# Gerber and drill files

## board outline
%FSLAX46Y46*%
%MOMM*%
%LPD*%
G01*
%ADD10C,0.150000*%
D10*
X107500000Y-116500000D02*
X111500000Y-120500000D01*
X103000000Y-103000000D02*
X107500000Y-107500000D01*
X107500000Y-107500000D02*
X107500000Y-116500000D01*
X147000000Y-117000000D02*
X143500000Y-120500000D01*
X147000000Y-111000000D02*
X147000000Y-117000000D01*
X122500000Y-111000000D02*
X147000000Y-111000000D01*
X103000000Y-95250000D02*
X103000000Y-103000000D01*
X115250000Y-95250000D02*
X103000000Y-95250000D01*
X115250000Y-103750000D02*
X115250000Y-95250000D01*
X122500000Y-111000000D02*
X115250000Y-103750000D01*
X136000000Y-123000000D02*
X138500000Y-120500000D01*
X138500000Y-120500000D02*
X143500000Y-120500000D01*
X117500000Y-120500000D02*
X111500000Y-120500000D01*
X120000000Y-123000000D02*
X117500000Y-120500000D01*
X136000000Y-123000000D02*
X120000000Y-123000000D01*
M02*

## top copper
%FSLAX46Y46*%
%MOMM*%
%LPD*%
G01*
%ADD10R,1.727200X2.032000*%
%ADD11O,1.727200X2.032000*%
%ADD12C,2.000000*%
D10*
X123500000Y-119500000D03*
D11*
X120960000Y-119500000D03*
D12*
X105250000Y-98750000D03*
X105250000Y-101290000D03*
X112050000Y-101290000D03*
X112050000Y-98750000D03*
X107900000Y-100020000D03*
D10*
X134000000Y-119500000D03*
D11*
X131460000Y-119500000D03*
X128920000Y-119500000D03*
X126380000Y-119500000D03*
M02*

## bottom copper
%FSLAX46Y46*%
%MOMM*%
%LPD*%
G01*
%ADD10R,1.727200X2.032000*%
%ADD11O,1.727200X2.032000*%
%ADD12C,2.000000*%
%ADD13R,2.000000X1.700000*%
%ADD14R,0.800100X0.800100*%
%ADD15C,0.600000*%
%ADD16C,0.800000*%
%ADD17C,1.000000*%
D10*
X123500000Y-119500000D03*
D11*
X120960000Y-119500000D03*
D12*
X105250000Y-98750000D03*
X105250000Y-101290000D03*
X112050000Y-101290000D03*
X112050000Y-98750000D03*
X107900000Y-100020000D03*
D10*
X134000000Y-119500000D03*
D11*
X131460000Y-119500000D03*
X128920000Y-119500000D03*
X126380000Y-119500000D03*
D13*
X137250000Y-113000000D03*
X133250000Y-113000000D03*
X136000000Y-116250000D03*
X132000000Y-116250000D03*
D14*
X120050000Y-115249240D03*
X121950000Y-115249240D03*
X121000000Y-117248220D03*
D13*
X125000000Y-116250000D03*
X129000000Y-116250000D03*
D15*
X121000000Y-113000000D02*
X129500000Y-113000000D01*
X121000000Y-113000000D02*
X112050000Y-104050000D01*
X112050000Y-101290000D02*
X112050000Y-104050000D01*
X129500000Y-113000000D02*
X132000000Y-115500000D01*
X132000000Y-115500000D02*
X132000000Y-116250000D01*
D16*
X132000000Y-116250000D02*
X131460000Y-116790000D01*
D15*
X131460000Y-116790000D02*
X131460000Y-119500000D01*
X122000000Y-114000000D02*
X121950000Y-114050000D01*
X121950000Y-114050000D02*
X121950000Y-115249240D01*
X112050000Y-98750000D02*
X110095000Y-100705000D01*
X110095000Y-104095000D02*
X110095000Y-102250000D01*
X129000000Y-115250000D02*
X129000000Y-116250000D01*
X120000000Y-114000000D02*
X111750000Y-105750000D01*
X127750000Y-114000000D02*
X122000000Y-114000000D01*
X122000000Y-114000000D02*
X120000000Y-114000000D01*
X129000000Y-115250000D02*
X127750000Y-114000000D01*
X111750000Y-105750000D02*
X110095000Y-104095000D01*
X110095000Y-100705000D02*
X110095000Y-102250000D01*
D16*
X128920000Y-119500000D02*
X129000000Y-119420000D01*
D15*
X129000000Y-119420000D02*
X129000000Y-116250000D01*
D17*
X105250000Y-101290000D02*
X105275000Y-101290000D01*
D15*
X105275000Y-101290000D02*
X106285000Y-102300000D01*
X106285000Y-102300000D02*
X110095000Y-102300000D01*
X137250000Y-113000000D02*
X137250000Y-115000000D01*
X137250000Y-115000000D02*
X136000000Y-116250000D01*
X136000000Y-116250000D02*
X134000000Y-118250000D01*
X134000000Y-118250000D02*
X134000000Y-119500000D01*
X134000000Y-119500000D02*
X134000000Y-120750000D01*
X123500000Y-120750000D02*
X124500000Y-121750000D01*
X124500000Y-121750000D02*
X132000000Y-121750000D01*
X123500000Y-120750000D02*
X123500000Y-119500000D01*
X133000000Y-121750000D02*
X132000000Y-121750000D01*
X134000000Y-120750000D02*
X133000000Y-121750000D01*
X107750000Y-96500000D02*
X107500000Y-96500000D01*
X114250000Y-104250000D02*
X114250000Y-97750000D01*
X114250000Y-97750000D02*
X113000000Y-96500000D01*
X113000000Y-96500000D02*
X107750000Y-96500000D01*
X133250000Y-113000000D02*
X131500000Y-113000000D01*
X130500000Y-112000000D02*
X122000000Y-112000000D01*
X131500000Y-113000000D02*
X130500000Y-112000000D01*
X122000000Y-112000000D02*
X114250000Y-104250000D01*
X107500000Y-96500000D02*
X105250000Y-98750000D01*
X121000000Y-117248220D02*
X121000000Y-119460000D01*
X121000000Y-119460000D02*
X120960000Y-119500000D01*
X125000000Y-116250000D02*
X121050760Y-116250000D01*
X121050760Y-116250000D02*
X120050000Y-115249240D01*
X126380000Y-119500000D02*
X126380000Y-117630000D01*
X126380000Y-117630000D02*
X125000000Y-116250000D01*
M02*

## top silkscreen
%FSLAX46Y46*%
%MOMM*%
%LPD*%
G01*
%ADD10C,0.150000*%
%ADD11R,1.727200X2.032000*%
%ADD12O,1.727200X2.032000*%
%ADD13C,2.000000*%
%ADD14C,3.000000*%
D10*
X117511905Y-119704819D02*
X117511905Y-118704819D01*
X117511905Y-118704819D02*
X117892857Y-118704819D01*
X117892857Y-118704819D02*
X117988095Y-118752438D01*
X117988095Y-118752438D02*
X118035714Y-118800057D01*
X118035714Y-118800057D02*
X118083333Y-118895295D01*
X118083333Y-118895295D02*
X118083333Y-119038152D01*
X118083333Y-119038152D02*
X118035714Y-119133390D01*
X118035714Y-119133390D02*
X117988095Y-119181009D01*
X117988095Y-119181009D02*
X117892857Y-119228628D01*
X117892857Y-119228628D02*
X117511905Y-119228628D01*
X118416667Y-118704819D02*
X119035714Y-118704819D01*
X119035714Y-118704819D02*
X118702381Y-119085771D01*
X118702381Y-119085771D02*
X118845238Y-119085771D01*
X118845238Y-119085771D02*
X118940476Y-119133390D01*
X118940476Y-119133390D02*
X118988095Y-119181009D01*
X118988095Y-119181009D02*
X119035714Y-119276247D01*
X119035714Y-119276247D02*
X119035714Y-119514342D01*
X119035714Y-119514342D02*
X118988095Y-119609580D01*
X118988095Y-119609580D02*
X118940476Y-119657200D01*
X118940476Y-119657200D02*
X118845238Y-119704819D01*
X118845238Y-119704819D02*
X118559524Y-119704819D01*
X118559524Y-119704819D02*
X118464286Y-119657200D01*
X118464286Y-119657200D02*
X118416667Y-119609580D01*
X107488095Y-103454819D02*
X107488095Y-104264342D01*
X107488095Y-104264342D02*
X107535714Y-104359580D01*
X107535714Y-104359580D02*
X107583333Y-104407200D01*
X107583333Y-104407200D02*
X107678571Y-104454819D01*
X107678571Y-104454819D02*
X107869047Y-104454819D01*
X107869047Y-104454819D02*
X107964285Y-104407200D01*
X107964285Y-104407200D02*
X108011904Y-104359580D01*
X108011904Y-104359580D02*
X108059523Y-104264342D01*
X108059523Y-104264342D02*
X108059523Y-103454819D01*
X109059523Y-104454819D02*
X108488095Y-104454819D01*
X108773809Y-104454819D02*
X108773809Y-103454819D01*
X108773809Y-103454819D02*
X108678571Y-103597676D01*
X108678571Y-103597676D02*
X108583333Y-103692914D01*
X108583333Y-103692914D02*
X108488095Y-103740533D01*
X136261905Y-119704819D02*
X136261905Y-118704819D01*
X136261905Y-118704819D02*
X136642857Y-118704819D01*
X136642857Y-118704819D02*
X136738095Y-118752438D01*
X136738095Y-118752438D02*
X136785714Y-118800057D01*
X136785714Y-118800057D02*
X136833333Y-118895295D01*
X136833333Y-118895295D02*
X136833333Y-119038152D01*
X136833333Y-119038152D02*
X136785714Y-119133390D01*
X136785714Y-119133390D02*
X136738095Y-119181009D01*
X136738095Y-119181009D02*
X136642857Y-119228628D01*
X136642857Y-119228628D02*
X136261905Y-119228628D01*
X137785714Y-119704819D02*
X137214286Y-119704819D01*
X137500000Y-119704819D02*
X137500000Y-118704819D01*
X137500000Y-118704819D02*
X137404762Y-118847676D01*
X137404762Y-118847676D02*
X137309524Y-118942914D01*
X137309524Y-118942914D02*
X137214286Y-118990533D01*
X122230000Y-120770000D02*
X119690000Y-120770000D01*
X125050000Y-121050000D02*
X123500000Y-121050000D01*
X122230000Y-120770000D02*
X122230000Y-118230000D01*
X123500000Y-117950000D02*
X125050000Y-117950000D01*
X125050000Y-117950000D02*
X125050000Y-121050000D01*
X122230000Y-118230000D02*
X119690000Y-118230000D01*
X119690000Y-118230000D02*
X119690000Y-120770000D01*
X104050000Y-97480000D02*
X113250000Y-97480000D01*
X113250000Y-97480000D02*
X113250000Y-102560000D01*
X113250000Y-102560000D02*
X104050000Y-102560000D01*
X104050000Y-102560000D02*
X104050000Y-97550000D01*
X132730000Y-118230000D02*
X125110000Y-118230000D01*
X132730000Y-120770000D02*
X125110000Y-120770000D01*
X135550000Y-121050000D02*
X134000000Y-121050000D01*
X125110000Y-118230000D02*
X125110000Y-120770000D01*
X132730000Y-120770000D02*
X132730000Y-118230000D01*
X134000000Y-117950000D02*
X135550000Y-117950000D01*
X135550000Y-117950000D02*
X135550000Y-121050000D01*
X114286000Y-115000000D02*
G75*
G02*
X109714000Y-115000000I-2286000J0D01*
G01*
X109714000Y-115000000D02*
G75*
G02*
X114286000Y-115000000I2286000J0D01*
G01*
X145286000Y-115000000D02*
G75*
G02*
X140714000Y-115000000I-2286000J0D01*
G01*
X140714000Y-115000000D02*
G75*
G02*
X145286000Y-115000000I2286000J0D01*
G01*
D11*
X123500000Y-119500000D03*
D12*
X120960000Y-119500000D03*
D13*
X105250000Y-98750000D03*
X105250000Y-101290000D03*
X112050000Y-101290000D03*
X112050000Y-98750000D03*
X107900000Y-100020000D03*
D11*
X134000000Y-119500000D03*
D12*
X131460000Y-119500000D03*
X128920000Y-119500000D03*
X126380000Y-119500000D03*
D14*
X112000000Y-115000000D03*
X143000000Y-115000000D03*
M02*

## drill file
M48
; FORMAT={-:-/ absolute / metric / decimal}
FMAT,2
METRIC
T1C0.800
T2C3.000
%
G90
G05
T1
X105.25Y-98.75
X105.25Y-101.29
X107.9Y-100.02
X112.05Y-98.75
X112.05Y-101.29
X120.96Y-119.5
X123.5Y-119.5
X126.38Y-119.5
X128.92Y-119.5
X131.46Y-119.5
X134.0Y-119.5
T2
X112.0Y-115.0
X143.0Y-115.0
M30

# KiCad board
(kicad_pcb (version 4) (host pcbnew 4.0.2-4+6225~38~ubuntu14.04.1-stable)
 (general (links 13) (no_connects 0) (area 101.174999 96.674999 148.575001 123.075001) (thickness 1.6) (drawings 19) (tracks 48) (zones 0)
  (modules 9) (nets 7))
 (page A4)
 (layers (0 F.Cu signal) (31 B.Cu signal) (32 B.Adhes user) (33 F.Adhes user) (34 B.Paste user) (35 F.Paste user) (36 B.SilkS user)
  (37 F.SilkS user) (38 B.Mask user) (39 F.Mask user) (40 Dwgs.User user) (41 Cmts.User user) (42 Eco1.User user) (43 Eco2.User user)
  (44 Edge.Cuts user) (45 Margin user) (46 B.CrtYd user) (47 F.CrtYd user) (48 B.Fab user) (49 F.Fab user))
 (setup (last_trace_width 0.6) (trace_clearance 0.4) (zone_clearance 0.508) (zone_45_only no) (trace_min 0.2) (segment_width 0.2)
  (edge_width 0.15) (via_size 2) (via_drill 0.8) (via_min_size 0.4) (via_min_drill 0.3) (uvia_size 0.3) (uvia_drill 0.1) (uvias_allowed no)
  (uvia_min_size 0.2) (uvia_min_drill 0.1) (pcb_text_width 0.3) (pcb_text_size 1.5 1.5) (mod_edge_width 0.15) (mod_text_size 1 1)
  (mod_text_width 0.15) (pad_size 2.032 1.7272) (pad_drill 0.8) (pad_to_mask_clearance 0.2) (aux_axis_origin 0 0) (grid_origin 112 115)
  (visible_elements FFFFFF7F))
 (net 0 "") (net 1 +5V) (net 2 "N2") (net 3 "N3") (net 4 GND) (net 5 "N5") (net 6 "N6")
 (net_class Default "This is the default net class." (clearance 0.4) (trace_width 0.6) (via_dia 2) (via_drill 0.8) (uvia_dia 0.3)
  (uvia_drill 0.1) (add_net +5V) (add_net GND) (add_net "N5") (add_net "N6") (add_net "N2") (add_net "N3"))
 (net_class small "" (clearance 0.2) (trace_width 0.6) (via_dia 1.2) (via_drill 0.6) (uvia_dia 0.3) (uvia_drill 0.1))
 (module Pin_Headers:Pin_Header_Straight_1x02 (layer F.Cu) (at 123.5 119.5 270)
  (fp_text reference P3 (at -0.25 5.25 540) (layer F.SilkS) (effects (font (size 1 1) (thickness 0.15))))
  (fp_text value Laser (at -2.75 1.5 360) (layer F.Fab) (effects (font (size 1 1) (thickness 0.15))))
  (fp_line (start 1.27 1.27) (end 1.27 3.81) (layer F.SilkS) (width 0.15))
  (fp_line (start 1.55 -1.55) (end 1.55 0) (layer F.SilkS) (width 0.15))
  (fp_line (start 1.27 1.27) (end -1.27 1.27) (layer F.SilkS) (width 0.15))
  (fp_line (start -1.55 0) (end -1.55 -1.55) (layer F.SilkS) (width 0.15))
  (fp_line (start -1.55 -1.55) (end 1.55 -1.55) (layer F.SilkS) (width 0.15))
  (fp_line (start -1.27 1.27) (end -1.27 3.81) (layer F.SilkS) (width 0.15))
  (fp_line (start -1.27 3.81) (end 1.27 3.81) (layer F.SilkS) (width 0.15))
  (pad 1 thru_hole rect (at 0 0 270) (size 2.032 1.7272) (drill 0.8) (layers *.Cu *.Mask F.SilkS) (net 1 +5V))
  (pad 2 thru_hole oval (at 0 2.54 270) (size 2.032 1.7272) (drill 0.8) (layers *.Cu *.Mask F.SilkS) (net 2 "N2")))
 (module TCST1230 (layer F.Cu) (at 105.25 98.75)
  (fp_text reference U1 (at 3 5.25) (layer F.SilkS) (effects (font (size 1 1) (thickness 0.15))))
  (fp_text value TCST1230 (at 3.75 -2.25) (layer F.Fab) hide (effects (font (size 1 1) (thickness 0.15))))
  (fp_line (start -1.2 -1.27) (end 8 -1.27) (layer F.SilkS) (width 0.15))
  (fp_line (start 8 -1.27) (end 8 3.81) (layer F.SilkS) (width 0.15))
  (fp_line (start 8 3.81) (end -1.2 3.81) (layer F.SilkS) (width 0.15))
  (fp_line (start -1.2 3.81) (end -1.2 -1.2) (layer F.SilkS) (width 0.15))
  (pad 1 thru_hole circle (at 0 0) (size 2 2) (drill 0.8) (layers *.Cu *.Mask F.SilkS) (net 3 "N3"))
  (pad 2 thru_hole circle (at 0 2.54) (size 2 2) (drill 0.8) (layers *.Cu *.Mask F.SilkS) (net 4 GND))
  (pad 3 thru_hole circle (at 6.8 2.54) (size 2 2) (drill 0.8) (layers *.Cu *.Mask F.SilkS) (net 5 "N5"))
  (pad 4 thru_hole circle (at 6.8 0) (size 2 2) (drill 0.8) (layers *.Cu *.Mask F.SilkS) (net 4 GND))
  (pad "" thru_hole circle (at 2.65 1.27) (size 2 2) (drill 0.8) (layers *.Cu *.Mask F.SilkS)))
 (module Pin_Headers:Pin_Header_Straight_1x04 (layer F.Cu) (at 134 119.5 270)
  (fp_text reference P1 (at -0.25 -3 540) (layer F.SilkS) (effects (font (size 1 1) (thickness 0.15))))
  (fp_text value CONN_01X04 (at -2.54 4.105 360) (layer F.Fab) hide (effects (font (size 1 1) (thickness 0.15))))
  (fp_line (start -1.27 1.27) (end -1.27 8.89) (layer F.SilkS) (width 0.15))
  (fp_line (start 1.27 1.27) (end 1.27 8.89) (layer F.SilkS) (width 0.15))
  (fp_line (start 1.55 -1.55) (end 1.55 0) (layer F.SilkS) (width 0.15))
  (fp_line (start -1.27 8.89) (end 1.27 8.89) (layer F.SilkS) (width 0.15))
  (fp_line (start 1.27 1.27) (end -1.27 1.27) (layer F.SilkS) (width 0.15))
  (fp_line (start -1.55 0) (end -1.55 -1.55) (layer F.SilkS) (width 0.15))
  (fp_line (start -1.55 -1.55) (end 1.55 -1.55) (layer F.SilkS) (width 0.15))
  (pad 1 thru_hole rect (at 0 0 270) (size 2.032 1.7272) (drill 0.8) (layers *.Cu *.Mask F.SilkS) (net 1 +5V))
  (pad 2 thru_hole oval (at 0 2.54 270) (size 2.032 1.7272) (drill 0.8) (layers *.Cu *.Mask F.SilkS) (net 5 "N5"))
  (pad 3 thru_hole oval (at 0 5.08 270) (size 2.032 1.7272) (drill 0.8) (layers *.Cu *.Mask F.SilkS) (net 4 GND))
  (pad 4 thru_hole oval (at 0 7.62 270) (size 2.032 1.7272) (drill 0.8) (layers *.Cu *.Mask F.SilkS) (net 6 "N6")))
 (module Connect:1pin (layer F.Cu) (at 112 115)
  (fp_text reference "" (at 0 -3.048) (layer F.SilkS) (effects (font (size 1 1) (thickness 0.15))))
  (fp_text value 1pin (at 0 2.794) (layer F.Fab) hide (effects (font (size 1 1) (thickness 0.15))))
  (fp_circle (center 0 0) (end 0 -2.286) (layer F.SilkS) (width 0.15))
  (pad "" np_thru_hole circle (at 0 0) (size 3 3) (drill 3) (layers *.Cu *.Mask F.SilkS)))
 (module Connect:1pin (layer F.Cu) (at 143 115)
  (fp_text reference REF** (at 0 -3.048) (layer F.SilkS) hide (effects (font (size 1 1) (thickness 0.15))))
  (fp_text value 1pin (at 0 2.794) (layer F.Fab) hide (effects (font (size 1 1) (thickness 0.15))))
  (fp_circle (center 0 0) (end 0 -2.286) (layer F.SilkS) (width 0.15))
  (pad "" np_thru_hole circle (at 0 0) (size 3 3) (drill 3) (layers *.Cu *.Mask F.SilkS)))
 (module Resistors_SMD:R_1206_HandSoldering (layer B.Cu) (at 135.25 113 180)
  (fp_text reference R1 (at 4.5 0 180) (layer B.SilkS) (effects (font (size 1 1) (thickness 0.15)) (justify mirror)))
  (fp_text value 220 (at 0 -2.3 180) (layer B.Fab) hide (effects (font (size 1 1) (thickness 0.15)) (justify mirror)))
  (pad 1 smd rect (at -2 0 180) (size 2 1.7) (layers B.Cu B.Paste B.Mask) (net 1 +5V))
  (pad 2 smd rect (at 2 0 180) (size 2 1.7) (layers B.Cu B.Paste B.Mask) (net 3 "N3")))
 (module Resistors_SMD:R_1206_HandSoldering (layer B.Cu) (at 134 116.25 180)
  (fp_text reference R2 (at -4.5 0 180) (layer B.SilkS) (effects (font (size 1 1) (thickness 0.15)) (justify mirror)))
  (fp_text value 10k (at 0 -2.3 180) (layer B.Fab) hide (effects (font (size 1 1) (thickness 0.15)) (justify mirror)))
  (pad 1 smd rect (at -2 0 180) (size 2 1.7) (layers B.Cu B.Paste B.Mask) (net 1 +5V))
  (pad 2 smd rect (at 2 0 180) (size 2 1.7) (layers B.Cu B.Paste B.Mask) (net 5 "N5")))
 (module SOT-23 (layer B.Cu) (at 121 116.25)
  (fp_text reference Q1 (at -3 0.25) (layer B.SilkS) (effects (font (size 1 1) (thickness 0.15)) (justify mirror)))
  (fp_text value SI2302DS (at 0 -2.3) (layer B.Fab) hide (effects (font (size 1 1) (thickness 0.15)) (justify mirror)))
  (pad 1 smd rect (at -0.95 -1.00076) (size 0.8001 0.8001) (layers B.Cu B.Paste B.Mask) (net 6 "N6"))
  (pad 2 smd rect (at 0.95 -1.00076) (size 0.8001 0.8001) (layers B.Cu B.Paste B.Mask) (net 4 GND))
  (pad 3 smd rect (at 0 0.99822) (size 0.8001 0.8001) (layers B.Cu B.Paste B.Mask) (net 2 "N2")))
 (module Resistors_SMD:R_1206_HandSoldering (layer B.Cu) (at 127 116.25)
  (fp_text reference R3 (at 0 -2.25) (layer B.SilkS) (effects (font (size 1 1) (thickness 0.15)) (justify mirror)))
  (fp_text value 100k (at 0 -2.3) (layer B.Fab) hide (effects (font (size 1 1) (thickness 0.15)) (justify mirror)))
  (pad 1 smd rect (at -2 0) (size 2 1.7) (layers B.Cu B.Paste B.Mask) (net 6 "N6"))
  (pad 2 smd rect (at 2 0) (size 2 1.7) (layers B.Cu B.Paste B.Mask) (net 4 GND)))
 (gr_line (start 107.5 116.5) (end 111.5 120.5) (angle 90) (layer Edge.Cuts) (width 0.15))
 (gr_line (start 103 103) (end 107.5 107.5) (angle 90) (layer Edge.Cuts) (width 0.15))
 (gr_line (start 107.5 107.5) (end 107.5 116.5) (angle 90) (layer Edge.Cuts) (width 0.15))
 (gr_line (start 147 117) (end 143.5 120.5) (angle 90) (layer Edge.Cuts) (width 0.15))
 (gr_line (start 147 111) (end 147 117) (angle 90) (layer Edge.Cuts) (width 0.15))
 (gr_line (start 122.5 111) (end 147 111) (angle 90) (layer Edge.Cuts) (width 0.15))
 (gr_line (start 103 95.25) (end 103 103) (angle 90) (layer Edge.Cuts) (width 0.15))
 (gr_line (start 115.25 95.25) (end 103 95.25) (angle 90) (layer Edge.Cuts) (width 0.15))
 (gr_line (start 115.25 103.75) (end 115.25 95.25) (angle 90) (layer Edge.Cuts) (width 0.15))
 (gr_line (start 122.5 111) (end 115.25 103.75) (angle 90) (layer Edge.Cuts) (width 0.15))
 (gr_line (start 136 123) (end 138.5 120.5) (angle 90) (layer Edge.Cuts) (width 0.15))
 (gr_line (start 138.5 120.5) (end 143.5 120.5) (angle 90) (layer Edge.Cuts) (width 0.15))
 (gr_line (start 117.5 120.5) (end 111.5 120.5) (angle 90) (layer Edge.Cuts) (width 0.15))
 (gr_line (start 120 123) (end 117.5 120.5) (angle 90) (layer Edge.Cuts) (width 0.15))
 (gr_line (start 136 123) (end 120 123) (angle 90) (layer Edge.Cuts) (width 0.15))
 (segment (start 121 113) (end 129.5 113) (width 0.6) (layer B.Cu) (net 5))
 (segment (start 121 113) (end 112.05 104.05) (width 0.6) (layer B.Cu) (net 5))
 (segment (start 112.05 101.29) (end 112.05 104.05) (width 0.6) (layer B.Cu) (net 5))
 (segment (start 129.5 113) (end 132 115.5) (width 0.6) (layer B.Cu) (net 5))
 (segment (start 132 115.5) (end 132 116.25) (width 0.6) (layer B.Cu) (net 5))
 (segment (start 132 116.25) (end 131.46 116.79) (width 0.8) (layer B.Cu) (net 5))
 (segment (start 131.46 116.79) (end 131.46 119.5) (width 0.6) (layer B.Cu) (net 5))
 (segment (start 122 114) (end 121.95 114.05) (width 0.6) (layer B.Cu) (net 4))
 (segment (start 121.95 114.05) (end 121.95 115.24924) (width 0.6) (layer B.Cu) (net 4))
 (segment (start 112.05 98.75) (end 110.095 100.705) (width 0.6) (layer B.Cu) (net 4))
 (segment (start 110.095 104.095) (end 110.095 102.25) (width 0.6) (layer B.Cu) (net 4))
 (segment (start 129 115.25) (end 129 116.25) (width 0.6) (layer B.Cu) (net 4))
 (segment (start 120 114) (end 111.75 105.75) (width 0.6) (layer B.Cu) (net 4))
 (segment (start 127.75 114) (end 122 114) (width 0.6) (layer B.Cu) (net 4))
 (segment (start 122 114) (end 120 114) (width 0.6) (layer B.Cu) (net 4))
 (segment (start 129 115.25) (end 127.75 114) (width 0.6) (layer B.Cu) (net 4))
 (segment (start 111.75 105.75) (end 110.095 104.095) (width 0.6) (layer B.Cu) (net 4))
 (segment (start 110.095 100.705) (end 110.095 102.25) (width 0.6) (layer B.Cu) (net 4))
 (segment (start 128.92 119.5) (end 129 119.42) (width 0.8) (layer B.Cu) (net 4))
 (segment (start 129 119.42) (end 129 116.25) (width 0.6) (layer B.Cu) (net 4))
 (segment (start 105.25 101.29) (end 105.275 101.29) (width 1) (layer B.Cu) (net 4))
 (segment (start 105.275 101.29) (end 106.285 102.3) (width 0.6) (layer B.Cu) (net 4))
 (segment (start 106.285 102.3) (end 110.095 102.3) (width 0.6) (layer B.Cu) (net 4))
 (segment (start 137.25 113) (end 137.25 115) (width 0.6) (layer B.Cu) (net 1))
 (segment (start 137.25 115) (end 136 116.25) (width 0.6) (layer B.Cu) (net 1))
 (segment (start 136 116.25) (end 134 118.25) (width 0.6) (layer B.Cu) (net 1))
 (segment (start 134 118.25) (end 134 119.5) (width 0.6) (layer B.Cu) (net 1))
 (segment (start 134 119.5) (end 134 120.75) (width 0.6) (layer B.Cu) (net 1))
 (segment (start 123.5 120.75) (end 124.5 121.75) (width 0.6) (layer B.Cu) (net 1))
 (segment (start 124.5 121.75) (end 132 121.75) (width 0.6) (layer B.Cu) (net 1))
 (segment (start 123.5 120.75) (end 123.5 119.5) (width 0.6) (layer B.Cu) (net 1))
 (segment (start 133 121.75) (end 132 121.75) (width 0.6) (layer B.Cu) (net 1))
 (segment (start 134 120.75) (end 133 121.75) (width 0.6) (layer B.Cu) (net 1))
 (segment (start 107.75 96.5) (end 107.5 96.5) (width 0.6) (layer B.Cu) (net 3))
 (segment (start 114.25 104.25) (end 114.25 97.75) (width 0.6) (layer B.Cu) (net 3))
 (segment (start 114.25 97.75) (end 113 96.5) (width 0.6) (layer B.Cu) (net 3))
 (segment (start 113 96.5) (end 107.75 96.5) (width 0.6) (layer B.Cu) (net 3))
 (segment (start 133.25 113) (end 131.5 113) (width 0.6) (layer B.Cu) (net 3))
 (segment (start 130.5 112) (end 122 112) (width 0.6) (layer B.Cu) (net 3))
 (segment (start 131.5 113) (end 130.5 112) (width 0.6) (layer B.Cu) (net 3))
 (segment (start 122 112) (end 114.25 104.25) (width 0.6) (layer B.Cu) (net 3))
 (segment (start 107.5 96.5) (end 105.25 98.75) (width 0.6) (layer B.Cu) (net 3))
 (segment (start 121 117.24822) (end 121 119.46) (width 0.6) (layer B.Cu) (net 2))
 (segment (start 121 119.46) (end 120.96 119.5) (width 0.6) (layer B.Cu) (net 2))
 (segment (start 125 116.25) (end 121.05076 116.25) (width 0.6) (layer B.Cu) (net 6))
 (segment (start 121.05076 116.25) (end 120.05 115.24924) (width 0.6) (layer B.Cu) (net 6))
 (segment (start 126.38 119.5) (end 126.38 117.63) (width 0.6) (layer B.Cu) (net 6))
 (segment (start 126.38 117.63) (end 125 116.25) (width 0.6) (layer B.Cu) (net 6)))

